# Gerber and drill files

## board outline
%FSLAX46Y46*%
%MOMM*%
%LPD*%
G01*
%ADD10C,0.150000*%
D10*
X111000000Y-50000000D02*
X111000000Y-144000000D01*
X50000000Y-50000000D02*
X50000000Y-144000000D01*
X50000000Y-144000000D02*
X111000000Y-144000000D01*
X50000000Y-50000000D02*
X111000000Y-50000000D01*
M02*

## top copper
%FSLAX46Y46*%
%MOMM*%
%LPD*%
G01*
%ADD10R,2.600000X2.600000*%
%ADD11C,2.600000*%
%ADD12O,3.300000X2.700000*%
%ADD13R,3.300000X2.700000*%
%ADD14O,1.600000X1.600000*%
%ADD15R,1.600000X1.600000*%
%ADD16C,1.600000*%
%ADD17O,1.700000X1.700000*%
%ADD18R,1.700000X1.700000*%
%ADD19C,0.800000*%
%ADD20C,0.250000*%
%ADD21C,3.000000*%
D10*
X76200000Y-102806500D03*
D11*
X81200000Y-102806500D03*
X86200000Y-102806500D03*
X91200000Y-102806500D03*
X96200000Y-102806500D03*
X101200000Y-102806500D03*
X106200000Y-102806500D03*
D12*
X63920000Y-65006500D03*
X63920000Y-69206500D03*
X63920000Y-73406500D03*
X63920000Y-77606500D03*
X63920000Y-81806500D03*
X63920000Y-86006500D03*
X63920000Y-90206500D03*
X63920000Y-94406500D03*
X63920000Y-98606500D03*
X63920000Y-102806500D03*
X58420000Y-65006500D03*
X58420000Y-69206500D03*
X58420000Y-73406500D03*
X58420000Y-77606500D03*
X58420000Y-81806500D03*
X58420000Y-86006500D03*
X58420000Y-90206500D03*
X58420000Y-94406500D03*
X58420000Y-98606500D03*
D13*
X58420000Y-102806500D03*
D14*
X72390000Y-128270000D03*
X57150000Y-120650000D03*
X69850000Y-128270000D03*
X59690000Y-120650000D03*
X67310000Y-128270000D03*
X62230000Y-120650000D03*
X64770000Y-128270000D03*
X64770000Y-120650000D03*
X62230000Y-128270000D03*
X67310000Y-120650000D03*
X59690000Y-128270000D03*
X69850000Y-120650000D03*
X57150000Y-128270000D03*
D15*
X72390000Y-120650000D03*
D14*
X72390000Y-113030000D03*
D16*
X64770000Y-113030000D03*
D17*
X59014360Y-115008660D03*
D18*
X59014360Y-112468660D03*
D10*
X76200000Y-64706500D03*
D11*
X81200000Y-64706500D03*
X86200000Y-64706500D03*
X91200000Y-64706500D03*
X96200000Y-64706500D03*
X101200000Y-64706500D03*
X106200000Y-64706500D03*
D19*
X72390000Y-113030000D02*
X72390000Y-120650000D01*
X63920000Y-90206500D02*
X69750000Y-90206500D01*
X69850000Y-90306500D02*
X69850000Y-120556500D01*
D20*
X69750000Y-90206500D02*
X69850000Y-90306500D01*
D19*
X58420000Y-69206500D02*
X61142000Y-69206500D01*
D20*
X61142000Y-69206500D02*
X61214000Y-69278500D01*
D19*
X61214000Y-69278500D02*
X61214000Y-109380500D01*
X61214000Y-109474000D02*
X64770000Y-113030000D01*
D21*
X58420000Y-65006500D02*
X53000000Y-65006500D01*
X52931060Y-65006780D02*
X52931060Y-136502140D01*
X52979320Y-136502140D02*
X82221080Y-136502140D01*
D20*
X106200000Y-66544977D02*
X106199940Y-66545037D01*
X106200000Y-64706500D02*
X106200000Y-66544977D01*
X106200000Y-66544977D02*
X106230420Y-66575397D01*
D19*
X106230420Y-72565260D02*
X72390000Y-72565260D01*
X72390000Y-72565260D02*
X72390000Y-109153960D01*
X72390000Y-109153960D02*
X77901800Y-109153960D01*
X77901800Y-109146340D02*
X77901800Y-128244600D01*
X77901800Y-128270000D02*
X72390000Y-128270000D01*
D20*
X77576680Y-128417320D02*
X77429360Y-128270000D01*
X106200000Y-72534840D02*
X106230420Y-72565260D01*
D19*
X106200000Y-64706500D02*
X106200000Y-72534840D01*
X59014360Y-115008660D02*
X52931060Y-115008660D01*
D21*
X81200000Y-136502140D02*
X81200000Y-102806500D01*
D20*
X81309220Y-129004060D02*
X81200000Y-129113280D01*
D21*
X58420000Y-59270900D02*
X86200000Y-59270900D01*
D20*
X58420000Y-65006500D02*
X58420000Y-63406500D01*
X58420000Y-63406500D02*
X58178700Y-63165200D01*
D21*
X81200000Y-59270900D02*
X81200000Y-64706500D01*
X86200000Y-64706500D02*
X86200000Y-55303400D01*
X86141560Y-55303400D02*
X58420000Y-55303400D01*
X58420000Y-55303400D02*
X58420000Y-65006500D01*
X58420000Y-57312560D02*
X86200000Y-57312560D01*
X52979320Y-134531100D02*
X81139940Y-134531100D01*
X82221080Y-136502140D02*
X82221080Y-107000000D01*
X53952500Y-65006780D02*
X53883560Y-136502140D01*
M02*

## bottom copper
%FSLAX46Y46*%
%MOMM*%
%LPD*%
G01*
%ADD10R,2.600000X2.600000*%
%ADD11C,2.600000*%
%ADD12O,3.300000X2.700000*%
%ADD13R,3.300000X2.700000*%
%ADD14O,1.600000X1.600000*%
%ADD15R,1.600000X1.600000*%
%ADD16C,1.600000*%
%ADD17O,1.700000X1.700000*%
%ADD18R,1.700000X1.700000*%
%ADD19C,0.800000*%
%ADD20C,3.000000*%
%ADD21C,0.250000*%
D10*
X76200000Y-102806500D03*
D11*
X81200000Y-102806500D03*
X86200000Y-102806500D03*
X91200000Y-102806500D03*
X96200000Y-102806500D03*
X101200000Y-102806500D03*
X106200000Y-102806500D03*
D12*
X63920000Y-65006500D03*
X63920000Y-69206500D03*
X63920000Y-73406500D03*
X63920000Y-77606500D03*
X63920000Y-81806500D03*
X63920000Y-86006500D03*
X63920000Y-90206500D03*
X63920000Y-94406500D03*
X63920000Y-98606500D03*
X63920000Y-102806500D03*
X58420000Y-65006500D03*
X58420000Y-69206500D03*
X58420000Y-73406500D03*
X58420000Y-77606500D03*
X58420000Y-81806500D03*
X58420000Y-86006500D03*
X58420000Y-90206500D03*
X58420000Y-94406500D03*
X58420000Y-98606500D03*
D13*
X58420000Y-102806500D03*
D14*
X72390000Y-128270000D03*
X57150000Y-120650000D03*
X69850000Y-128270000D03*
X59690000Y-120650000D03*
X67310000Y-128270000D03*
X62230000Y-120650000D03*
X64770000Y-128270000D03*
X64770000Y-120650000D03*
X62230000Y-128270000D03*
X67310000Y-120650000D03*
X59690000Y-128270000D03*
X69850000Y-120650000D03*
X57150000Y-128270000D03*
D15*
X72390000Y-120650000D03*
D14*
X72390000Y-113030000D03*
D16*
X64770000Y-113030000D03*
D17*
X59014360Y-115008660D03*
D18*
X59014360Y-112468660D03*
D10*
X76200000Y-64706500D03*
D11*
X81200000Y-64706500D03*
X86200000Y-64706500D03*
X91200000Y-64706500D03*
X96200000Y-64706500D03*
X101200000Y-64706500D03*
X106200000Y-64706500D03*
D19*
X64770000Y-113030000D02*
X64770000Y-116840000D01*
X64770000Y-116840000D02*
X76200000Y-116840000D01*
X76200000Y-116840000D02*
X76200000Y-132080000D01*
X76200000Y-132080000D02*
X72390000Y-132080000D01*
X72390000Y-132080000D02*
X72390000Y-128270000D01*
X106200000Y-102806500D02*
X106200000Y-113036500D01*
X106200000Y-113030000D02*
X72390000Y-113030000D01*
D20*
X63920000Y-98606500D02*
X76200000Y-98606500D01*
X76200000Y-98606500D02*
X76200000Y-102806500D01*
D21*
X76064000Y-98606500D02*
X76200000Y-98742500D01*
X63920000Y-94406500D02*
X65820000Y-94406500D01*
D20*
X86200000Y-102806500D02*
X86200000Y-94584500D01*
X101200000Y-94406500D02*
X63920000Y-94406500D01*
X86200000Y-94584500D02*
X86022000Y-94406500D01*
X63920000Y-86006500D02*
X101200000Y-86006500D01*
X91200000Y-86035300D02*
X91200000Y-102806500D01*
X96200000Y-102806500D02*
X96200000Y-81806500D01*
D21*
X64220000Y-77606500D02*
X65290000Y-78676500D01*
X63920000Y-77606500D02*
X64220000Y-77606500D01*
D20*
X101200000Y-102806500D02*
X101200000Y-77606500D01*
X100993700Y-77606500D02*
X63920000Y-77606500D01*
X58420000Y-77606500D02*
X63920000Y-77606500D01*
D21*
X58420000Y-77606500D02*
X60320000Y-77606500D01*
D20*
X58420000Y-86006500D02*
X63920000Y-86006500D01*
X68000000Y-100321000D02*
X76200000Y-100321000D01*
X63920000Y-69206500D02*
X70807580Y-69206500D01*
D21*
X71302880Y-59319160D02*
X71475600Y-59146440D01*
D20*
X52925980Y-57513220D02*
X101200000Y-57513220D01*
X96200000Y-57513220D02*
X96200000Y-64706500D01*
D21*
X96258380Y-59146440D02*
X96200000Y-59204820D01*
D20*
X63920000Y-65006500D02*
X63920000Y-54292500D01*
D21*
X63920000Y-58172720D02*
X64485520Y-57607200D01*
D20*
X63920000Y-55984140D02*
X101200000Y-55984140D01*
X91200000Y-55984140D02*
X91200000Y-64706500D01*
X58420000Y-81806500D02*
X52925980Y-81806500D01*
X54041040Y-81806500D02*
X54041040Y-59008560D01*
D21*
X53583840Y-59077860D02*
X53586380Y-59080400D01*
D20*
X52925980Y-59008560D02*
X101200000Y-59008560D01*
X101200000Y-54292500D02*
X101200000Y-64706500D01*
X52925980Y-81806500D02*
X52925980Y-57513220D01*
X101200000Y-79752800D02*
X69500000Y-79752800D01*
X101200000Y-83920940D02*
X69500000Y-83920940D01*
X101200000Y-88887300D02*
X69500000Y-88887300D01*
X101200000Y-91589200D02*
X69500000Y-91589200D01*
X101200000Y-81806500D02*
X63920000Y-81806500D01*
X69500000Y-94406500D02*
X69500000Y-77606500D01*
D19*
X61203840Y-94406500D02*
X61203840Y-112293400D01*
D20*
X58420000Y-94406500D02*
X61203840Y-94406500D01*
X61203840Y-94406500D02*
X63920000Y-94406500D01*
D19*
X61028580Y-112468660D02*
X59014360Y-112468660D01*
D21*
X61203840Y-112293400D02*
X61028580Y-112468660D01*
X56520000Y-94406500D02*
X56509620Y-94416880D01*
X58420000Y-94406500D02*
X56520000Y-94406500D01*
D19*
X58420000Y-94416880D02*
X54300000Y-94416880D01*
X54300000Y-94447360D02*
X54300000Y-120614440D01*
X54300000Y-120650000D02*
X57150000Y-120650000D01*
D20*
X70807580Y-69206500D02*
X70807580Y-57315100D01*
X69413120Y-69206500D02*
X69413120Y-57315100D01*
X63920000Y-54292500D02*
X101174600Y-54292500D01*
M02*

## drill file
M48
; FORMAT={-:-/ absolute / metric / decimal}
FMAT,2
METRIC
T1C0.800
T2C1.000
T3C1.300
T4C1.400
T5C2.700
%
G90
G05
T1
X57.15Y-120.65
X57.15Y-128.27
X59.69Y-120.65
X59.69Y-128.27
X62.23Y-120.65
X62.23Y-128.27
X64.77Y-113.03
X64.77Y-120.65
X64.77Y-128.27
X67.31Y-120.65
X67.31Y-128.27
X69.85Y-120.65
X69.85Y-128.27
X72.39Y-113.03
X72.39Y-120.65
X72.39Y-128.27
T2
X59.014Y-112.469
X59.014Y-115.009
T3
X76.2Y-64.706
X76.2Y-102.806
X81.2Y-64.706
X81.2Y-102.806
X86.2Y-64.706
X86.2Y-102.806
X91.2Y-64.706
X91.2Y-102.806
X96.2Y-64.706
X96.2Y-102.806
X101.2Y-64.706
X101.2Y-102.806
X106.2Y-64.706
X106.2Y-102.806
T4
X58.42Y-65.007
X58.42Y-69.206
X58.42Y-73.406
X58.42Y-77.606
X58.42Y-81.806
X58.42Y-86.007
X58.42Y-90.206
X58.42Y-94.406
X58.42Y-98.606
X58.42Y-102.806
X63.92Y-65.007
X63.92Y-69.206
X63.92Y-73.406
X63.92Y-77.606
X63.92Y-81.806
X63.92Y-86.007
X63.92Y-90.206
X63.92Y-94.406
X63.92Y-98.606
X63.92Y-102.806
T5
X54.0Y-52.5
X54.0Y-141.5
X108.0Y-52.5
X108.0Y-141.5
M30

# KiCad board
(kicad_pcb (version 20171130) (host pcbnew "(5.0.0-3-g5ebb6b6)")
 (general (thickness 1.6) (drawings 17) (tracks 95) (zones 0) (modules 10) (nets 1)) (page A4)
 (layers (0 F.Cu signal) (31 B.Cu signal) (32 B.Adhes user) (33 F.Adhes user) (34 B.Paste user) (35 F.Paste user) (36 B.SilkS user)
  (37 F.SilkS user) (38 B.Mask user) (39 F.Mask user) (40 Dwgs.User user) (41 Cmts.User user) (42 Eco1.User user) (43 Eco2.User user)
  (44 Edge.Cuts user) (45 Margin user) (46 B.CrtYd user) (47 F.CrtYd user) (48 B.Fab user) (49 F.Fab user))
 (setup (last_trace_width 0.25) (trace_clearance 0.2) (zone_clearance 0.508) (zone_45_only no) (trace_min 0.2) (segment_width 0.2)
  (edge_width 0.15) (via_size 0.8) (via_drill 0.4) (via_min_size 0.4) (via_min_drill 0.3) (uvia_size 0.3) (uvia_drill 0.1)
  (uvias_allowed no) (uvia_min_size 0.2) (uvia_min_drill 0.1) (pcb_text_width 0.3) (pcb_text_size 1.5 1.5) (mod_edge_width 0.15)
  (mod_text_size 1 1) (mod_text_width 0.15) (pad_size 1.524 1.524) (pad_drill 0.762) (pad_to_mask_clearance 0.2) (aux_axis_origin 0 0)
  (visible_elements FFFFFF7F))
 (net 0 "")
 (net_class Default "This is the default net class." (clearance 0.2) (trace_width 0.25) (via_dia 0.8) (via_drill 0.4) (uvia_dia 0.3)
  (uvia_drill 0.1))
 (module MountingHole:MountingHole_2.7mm (layer F.Cu) (at 54 52.5)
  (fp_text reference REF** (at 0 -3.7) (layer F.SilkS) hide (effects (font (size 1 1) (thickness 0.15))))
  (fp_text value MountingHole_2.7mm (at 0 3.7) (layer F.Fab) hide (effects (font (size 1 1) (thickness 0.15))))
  (pad 1 np_thru_hole circle (at 0 0) (size 2.7 2.7) (drill 2.7) (layers *.Cu *.Mask)))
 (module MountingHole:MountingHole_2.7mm (layer F.Cu) (at 54 141.5)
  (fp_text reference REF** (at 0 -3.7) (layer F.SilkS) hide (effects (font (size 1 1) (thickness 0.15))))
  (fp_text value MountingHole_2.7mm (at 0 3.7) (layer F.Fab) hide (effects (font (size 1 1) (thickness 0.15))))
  (pad 1 np_thru_hole circle (at 0 0) (size 2.7 2.7) (drill 2.7) (layers *.Cu *.Mask)))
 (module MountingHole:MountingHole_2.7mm (layer F.Cu) (at 108 141.5)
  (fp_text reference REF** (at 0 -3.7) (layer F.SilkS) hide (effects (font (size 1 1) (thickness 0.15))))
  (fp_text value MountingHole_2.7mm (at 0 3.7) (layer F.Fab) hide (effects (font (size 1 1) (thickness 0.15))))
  (pad 1 np_thru_hole circle (at 0 0) (size 2.7 2.7) (drill 2.7) (layers *.Cu *.Mask)))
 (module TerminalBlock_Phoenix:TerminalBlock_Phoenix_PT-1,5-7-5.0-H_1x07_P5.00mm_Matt (layer F.Cu) (at 76.2 102.8065)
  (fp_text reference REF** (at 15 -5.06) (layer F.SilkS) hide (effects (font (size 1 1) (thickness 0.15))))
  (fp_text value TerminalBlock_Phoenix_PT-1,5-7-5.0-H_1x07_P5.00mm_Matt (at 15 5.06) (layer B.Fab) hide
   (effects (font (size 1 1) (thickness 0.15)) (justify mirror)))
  (pad 1 thru_hole rect (at 0 0) (size 2.6 2.6) (drill 1.3) (layers *.Cu *.Mask))
  (pad 2 thru_hole circle (at 5 0) (size 2.6 2.6) (drill 1.3) (layers *.Cu *.Mask))
  (pad 3 thru_hole circle (at 10 0) (size 2.6 2.6) (drill 1.3) (layers *.Cu *.Mask))
  (pad 4 thru_hole circle (at 15 0) (size 2.6 2.6) (drill 1.3) (layers *.Cu *.Mask))
  (pad 5 thru_hole circle (at 20 0) (size 2.6 2.6) (drill 1.3) (layers *.Cu *.Mask))
  (pad 6 thru_hole circle (at 25 0) (size 2.6 2.6) (drill 1.3) (layers *.Cu *.Mask))
  (pad 7 thru_hole circle (at 30 0) (size 2.6 2.6) (drill 1.3) (layers *.Cu *.Mask)))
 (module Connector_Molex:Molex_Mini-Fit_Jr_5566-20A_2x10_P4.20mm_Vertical (layer F.Cu) (at 58.42 102.8065 90)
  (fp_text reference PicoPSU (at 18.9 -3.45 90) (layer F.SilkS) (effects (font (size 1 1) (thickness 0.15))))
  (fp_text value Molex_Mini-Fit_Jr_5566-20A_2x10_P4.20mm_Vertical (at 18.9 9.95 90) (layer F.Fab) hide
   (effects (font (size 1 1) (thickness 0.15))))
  (pad 20 thru_hole oval (at 37.8 5.5 90) (size 2.7 3.3) (drill 1.4) (layers *.Cu *.Mask))
  (pad 19 thru_hole oval (at 33.6 5.5 90) (size 2.7 3.3) (drill 1.4) (layers *.Cu *.Mask))
  (pad 18 thru_hole oval (at 29.4 5.5 90) (size 2.7 3.3) (drill 1.4) (layers *.Cu *.Mask))
  (pad 17 thru_hole oval (at 25.2 5.5 90) (size 2.7 3.3) (drill 1.4) (layers *.Cu *.Mask))
  (pad 16 thru_hole oval (at 21 5.5 90) (size 2.7 3.3) (drill 1.4) (layers *.Cu *.Mask))
  (pad 15 thru_hole oval (at 16.8 5.5 90) (size 2.7 3.3) (drill 1.4) (layers *.Cu *.Mask))
  (pad 14 thru_hole oval (at 12.6 5.5 90) (size 2.7 3.3) (drill 1.4) (layers *.Cu *.Mask))
  (pad 13 thru_hole oval (at 8.4 5.5 90) (size 2.7 3.3) (drill 1.4) (layers *.Cu *.Mask))
  (pad 12 thru_hole oval (at 4.2 5.5 90) (size 2.7 3.3) (drill 1.4) (layers *.Cu *.Mask))
  (pad 11 thru_hole oval (at 0 5.5 90) (size 2.7 3.3) (drill 1.4) (layers *.Cu *.Mask))
  (pad 10 thru_hole oval (at 37.8 0 90) (size 2.7 3.3) (drill 1.4) (layers *.Cu *.Mask))
  (pad 9 thru_hole oval (at 33.6 0 90) (size 2.7 3.3) (drill 1.4) (layers *.Cu *.Mask))
  (pad 8 thru_hole oval (at 29.4 0 90) (size 2.7 3.3) (drill 1.4) (layers *.Cu *.Mask))
  (pad 7 thru_hole oval (at 25.2 0 90) (size 2.7 3.3) (drill 1.4) (layers *.Cu *.Mask))
  (pad 6 thru_hole oval (at 21 0 90) (size 2.7 3.3) (drill 1.4) (layers *.Cu *.Mask))
  (pad 5 thru_hole oval (at 16.8 0 90) (size 2.7 3.3) (drill 1.4) (layers *.Cu *.Mask))
  (pad 4 thru_hole oval (at 12.6 0 90) (size 2.7 3.3) (drill 1.4) (layers *.Cu *.Mask))
  (pad 3 thru_hole oval (at 8.4 0 90) (size 2.7 3.3) (drill 1.4) (layers *.Cu *.Mask))
  (pad 2 thru_hole oval (at 4.2 0 90) (size 2.7 3.3) (drill 1.4) (layers *.Cu *.Mask))
  (pad 1 thru_hole rect (at 0 0 90) (size 2.7 3.3) (drill 1.4) (layers *.Cu *.Mask)))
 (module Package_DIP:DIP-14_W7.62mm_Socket (layer F.Cu) (at 72.39 120.65 270)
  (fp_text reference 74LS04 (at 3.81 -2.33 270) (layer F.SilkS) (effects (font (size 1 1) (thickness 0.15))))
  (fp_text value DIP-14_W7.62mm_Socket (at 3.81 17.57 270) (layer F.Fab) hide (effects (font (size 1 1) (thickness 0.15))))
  (pad 14 thru_hole oval (at 7.62 0 270) (size 1.6 1.6) (drill 0.8) (layers *.Cu *.Mask))
  (pad 7 thru_hole oval (at 0 15.24 270) (size 1.6 1.6) (drill 0.8) (layers *.Cu *.Mask))
  (pad 13 thru_hole oval (at 7.62 2.54 270) (size 1.6 1.6) (drill 0.8) (layers *.Cu *.Mask))
  (pad 6 thru_hole oval (at 0 12.7 270) (size 1.6 1.6) (drill 0.8) (layers *.Cu *.Mask))
  (pad 12 thru_hole oval (at 7.62 5.08 270) (size 1.6 1.6) (drill 0.8) (layers *.Cu *.Mask))
  (pad 5 thru_hole oval (at 0 10.16 270) (size 1.6 1.6) (drill 0.8) (layers *.Cu *.Mask))
  (pad 11 thru_hole oval (at 7.62 7.62 270) (size 1.6 1.6) (drill 0.8) (layers *.Cu *.Mask))
  (pad 4 thru_hole oval (at 0 7.62 270) (size 1.6 1.6) (drill 0.8) (layers *.Cu *.Mask))
  (pad 10 thru_hole oval (at 7.62 10.16 270) (size 1.6 1.6) (drill 0.8) (layers *.Cu *.Mask))
  (pad 3 thru_hole oval (at 0 5.08 270) (size 1.6 1.6) (drill 0.8) (layers *.Cu *.Mask))
  (pad 9 thru_hole oval (at 7.62 12.7 270) (size 1.6 1.6) (drill 0.8) (layers *.Cu *.Mask))
  (pad 2 thru_hole oval (at 0 2.54 270) (size 1.6 1.6) (drill 0.8) (layers *.Cu *.Mask))
  (pad 8 thru_hole oval (at 7.62 15.24 270) (size 1.6 1.6) (drill 0.8) (layers *.Cu *.Mask))
  (pad 1 thru_hole rect (at 0 0 270) (size 1.6 1.6) (drill 0.8) (layers *.Cu *.Mask)))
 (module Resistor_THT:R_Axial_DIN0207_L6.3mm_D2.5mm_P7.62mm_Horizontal (layer F.Cu) (at 64.77 113.03)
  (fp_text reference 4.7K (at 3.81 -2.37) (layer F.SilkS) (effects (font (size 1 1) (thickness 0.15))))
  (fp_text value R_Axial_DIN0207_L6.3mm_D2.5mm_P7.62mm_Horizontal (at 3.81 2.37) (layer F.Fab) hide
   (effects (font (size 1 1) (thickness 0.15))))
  (pad 2 thru_hole oval (at 7.62 0) (size 1.6 1.6) (drill 0.8) (layers *.Cu *.Mask))
  (pad 1 thru_hole circle (at 0 0) (size 1.6 1.6) (drill 0.8) (layers *.Cu *.Mask)))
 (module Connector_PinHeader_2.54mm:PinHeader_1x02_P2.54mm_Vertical (layer F.Cu) (at 59.01436 112.46866)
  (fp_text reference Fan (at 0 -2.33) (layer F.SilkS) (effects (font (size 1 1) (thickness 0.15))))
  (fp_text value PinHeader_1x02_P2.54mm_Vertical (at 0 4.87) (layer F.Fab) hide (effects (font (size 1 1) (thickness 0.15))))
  (pad 2 thru_hole oval (at 0 2.54) (size 1.7 1.7) (drill 1) (layers *.Cu *.Mask))
  (pad 1 thru_hole rect (at 0 0) (size 1.7 1.7) (drill 1) (layers *.Cu *.Mask)))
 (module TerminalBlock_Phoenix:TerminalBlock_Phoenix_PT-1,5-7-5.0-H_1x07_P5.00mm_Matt (layer F.Cu) (at 76.2 64.7065)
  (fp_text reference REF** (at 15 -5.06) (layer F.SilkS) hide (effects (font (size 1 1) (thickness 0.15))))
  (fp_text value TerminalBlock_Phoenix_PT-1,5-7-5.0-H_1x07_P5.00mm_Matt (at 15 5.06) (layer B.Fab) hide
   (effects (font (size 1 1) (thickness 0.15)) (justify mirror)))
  (pad 1 thru_hole rect (at 0 0) (size 2.6 2.6) (drill 1.3) (layers *.Cu *.Mask))
  (pad 2 thru_hole circle (at 5 0) (size 2.6 2.6) (drill 1.3) (layers *.Cu *.Mask))
  (pad 3 thru_hole circle (at 10 0) (size 2.6 2.6) (drill 1.3) (layers *.Cu *.Mask))
  (pad 4 thru_hole circle (at 15 0) (size 2.6 2.6) (drill 1.3) (layers *.Cu *.Mask))
  (pad 5 thru_hole circle (at 20 0) (size 2.6 2.6) (drill 1.3) (layers *.Cu *.Mask))
  (pad 6 thru_hole circle (at 25 0) (size 2.6 2.6) (drill 1.3) (layers *.Cu *.Mask))
  (pad 7 thru_hole circle (at 30 0) (size 2.6 2.6) (drill 1.3) (layers *.Cu *.Mask)))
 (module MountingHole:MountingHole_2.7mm (layer F.Cu) (at 108 52.5)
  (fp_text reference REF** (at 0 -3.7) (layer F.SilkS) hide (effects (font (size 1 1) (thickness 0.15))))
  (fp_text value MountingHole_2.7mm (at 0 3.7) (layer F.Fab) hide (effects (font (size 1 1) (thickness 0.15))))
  (pad 1 np_thru_hole circle (at 0 0) (size 2.7 2.7) (drill 2.7) (layers *.Cu *.Mask)))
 (gr_line (start 111 50) (end 111 144) (layer Edge.Cuts) (width 0.15))
 (gr_line (start 50 50) (end 50 144) (layer Edge.Cuts) (width 0.15))
 (gr_line (start 50 144) (end 111 144) (layer Edge.Cuts) (width 0.15))
 (gr_line (start 50 50) (end 111 50) (layer Edge.Cuts) (width 0.15))
 (segment (start 72.39 113.03) (end 72.39 120.65) (width 0.8) (layer F.Cu) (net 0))
 (segment (start 63.92 90.2065) (end 69.75 90.2065) (width 0.8) (layer F.Cu) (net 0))
 (segment (start 69.85 90.3065) (end 69.85 120.5565) (width 0.8) (layer F.Cu) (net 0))
 (segment (start 69.75 90.2065) (end 69.85 90.3065) (width 0.25) (layer F.Cu) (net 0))
 (segment (start 64.77 113.03) (end 64.77 116.84) (width 0.8) (layer B.Cu) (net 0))
 (segment (start 64.77 116.84) (end 76.2 116.84) (width 0.8) (layer B.Cu) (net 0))
 (segment (start 76.2 116.84) (end 76.2 132.08) (width 0.8) (layer B.Cu) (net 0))
 (segment (start 76.2 132.08) (end 72.39 132.08) (width 0.8) (layer B.Cu) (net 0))
 (segment (start 72.39 132.08) (end 72.39 128.27) (width 0.8) (layer B.Cu) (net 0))
 (segment (start 106.2 102.8065) (end 106.2 113.0365) (width 0.8) (layer B.Cu) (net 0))
 (segment (start 106.2 113.03) (end 72.39 113.03) (width 0.8) (layer B.Cu) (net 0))
 (segment (start 58.42 69.2065) (end 61.142 69.2065) (width 0.8) (layer F.Cu) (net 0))
 (segment (start 61.142 69.2065) (end 61.214 69.2785) (width 0.25) (layer F.Cu) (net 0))
 (segment (start 61.214 69.2785) (end 61.214 109.3805) (width 0.8) (layer F.Cu) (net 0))
 (segment (start 61.214 109.474) (end 64.77 113.03) (width 0.8) (layer F.Cu) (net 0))
 (segment (start 63.92 98.6065) (end 76.2 98.6065) (width 3) (layer B.Cu) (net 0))
 (segment (start 76.2 98.6065) (end 76.2 102.8065) (width 3) (layer B.Cu) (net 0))
 (segment (start 76.064 98.6065) (end 76.2 98.7425) (width 0.25) (layer B.Cu) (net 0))
 (segment (start 63.92 94.4065) (end 65.82 94.4065) (width 0.25) (layer B.Cu) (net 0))
 (segment (start 86.2 102.8065) (end 86.2 94.5845) (width 3) (layer B.Cu) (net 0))
 (segment (start 101.2 94.4065) (end 63.92 94.4065) (width 3) (layer B.Cu) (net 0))
 (segment (start 86.2 94.5845) (end 86.022 94.4065) (width 3) (layer B.Cu) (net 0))
 (segment (start 63.92 86.0065) (end 101.2 86.0065) (width 3) (layer B.Cu) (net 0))
 (segment (start 91.2 86.0353) (end 91.2 102.8065) (width 3) (layer B.Cu) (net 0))
 (segment (start 96.2 102.8065) (end 96.2 81.8065) (width 3) (layer B.Cu) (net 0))
 (segment (start 64.22 77.6065) (end 65.29 78.6765) (width 0.25) (layer B.Cu) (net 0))
 (segment (start 63.92 77.6065) (end 64.22 77.6065) (width 0.25) (layer B.Cu) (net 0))
 (segment (start 101.2 102.8065) (end 101.2 77.6065) (width 3) (layer B.Cu) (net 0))
 (segment (start 100.9937 77.6065) (end 63.92 77.6065) (width 3) (layer B.Cu) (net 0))
 (segment (start 58.42 65.0065) (end 53 65.0065) (width 3) (layer F.Cu) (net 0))
 (segment (start 52.93106 65.00678) (end 52.93106 136.50214) (width 3) (layer F.Cu) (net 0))
 (segment (start 52.97932 136.50214) (end 82.22108 136.50214) (width 3) (layer F.Cu) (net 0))
 (segment (start 106.2 66.544977) (end 106.19994 66.545037) (width 0.25) (layer F.Cu) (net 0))
 (segment (start 106.2 64.7065) (end 106.2 66.544977) (width 0.25) (layer F.Cu) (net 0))
 (segment (start 106.2 66.544977) (end 106.23042 66.575397) (width 0.25) (layer F.Cu) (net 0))
 (segment (start 106.23042 72.56526) (end 72.39 72.56526) (width 0.8) (layer F.Cu) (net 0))
 (segment (start 72.39 72.56526) (end 72.39 109.15396) (width 0.8) (layer F.Cu) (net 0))
 (segment (start 72.39 109.15396) (end 77.9018 109.15396) (width 0.8) (layer F.Cu) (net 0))
 (segment (start 77.9018 109.14634) (end 77.9018 128.2446) (width 0.8) (layer F.Cu) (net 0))
 (segment (start 77.9018 128.27) (end 72.39 128.27) (width 0.8) (layer F.Cu) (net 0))
 (segment (start 77.57668 128.41732) (end 77.42936 128.27) (width 0.25) (layer F.Cu) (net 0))
 (segment (start 106.2 72.53484) (end 106.23042 72.56526) (width 0.25) (layer F.Cu) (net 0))
 (segment (start 106.2 64.7065) (end 106.2 72.53484) (width 0.8) (layer F.Cu) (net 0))
 (segment (start 59.01436 115.00866) (end 52.93106 115.00866) (width 0.8) (layer F.Cu) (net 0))
 (segment (start 81.2 136.50214) (end 81.2 102.8065) (width 3) (layer F.Cu) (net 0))
 (segment (start 81.30922 129.00406) (end 81.2 129.11328) (width 0.25) (layer F.Cu) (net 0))
 (segment (start 58.42 59.2709) (end 86.2 59.2709) (width 3) (layer F.Cu) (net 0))
 (segment (start 58.42 65.0065) (end 58.42 63.4065) (width 0.25) (layer F.Cu) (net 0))
 (segment (start 58.42 63.4065) (end 58.1787 63.1652) (width 0.25) (layer F.Cu) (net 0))
 (segment (start 81.2 59.2709) (end 81.2 64.7065) (width 3) (layer F.Cu) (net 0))
 (segment (start 86.2 64.7065) (end 86.2 55.3034) (width 3) (layer F.Cu) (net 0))
 (segment (start 86.14156 55.3034) (end 58.42 55.3034) (width 3) (layer F.Cu) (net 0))
 (segment (start 58.42 55.3034) (end 58.42 65.0065) (width 3) (layer F.Cu) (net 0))
 (segment (start 58.42 57.31256) (end 86.2 57.31256) (width 3) (layer F.Cu) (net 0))
 (segment (start 52.97932 134.5311) (end 81.13994 134.5311) (width 3) (layer F.Cu) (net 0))
 (segment (start 82.22108 136.50214) (end 82.22108 107) (width 3) (layer F.Cu) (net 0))
 (segment (start 53.9525 65.00678) (end 53.88356 136.50214) (width 3) (layer F.Cu) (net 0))
 (segment (start 58.42 77.6065) (end 63.92 77.6065) (width 3) (layer B.Cu) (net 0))
 (segment (start 58.42 77.6065) (end 60.32 77.6065) (width 0.25) (layer B.Cu) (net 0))
 (segment (start 58.42 86.0065) (end 63.92 86.0065) (width 3) (layer B.Cu) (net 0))
 (segment (start 68 100.321) (end 76.2 100.321) (width 3) (layer B.Cu) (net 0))
 (segment (start 63.92 69.2065) (end 70.80758 69.2065) (width 3) (layer B.Cu) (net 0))
 (segment (start 71.30288 59.31916) (end 71.4756 59.14644) (width 0.25) (layer B.Cu) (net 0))
 (segment (start 52.92598 57.51322) (end 101.2 57.51322) (width 3) (layer B.Cu) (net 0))
 (segment (start 96.2 57.51322) (end 96.2 64.7065) (width 3) (layer B.Cu) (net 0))
 (segment (start 96.25838 59.14644) (end 96.2 59.20482) (width 0.25) (layer B.Cu) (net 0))
 (segment (start 63.92 65.0065) (end 63.92 54.2925) (width 3) (layer B.Cu) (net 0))
 (segment (start 63.92 58.17272) (end 64.48552 57.6072) (width 0.25) (layer B.Cu) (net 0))
 (segment (start 63.92 55.98414) (end 101.2 55.98414) (width 3) (layer B.Cu) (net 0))
 (segment (start 91.2 55.98414) (end 91.2 64.7065) (width 3) (layer B.Cu) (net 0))
 (segment (start 58.42 81.8065) (end 52.92598 81.8065) (width 3) (layer B.Cu) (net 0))
 (segment (start 54.04104 81.8065) (end 54.04104 59.00856) (width 3) (layer B.Cu) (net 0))
 (segment (start 53.58384 59.07786) (end 53.58638 59.0804) (width 0.25) (layer B.Cu) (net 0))
 (segment (start 52.92598 59.00856) (end 101.2 59.00856) (width 3) (layer B.Cu) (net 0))
 (segment (start 101.2 54.2925) (end 101.2 64.7065) (width 3) (layer B.Cu) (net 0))
 (segment (start 52.92598 81.8065) (end 52.92598 57.51322) (width 3) (layer B.Cu) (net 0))
 (segment (start 101.2 79.7528) (end 69.5 79.7528) (width 3) (layer B.Cu) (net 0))
 (segment (start 101.2 83.92094) (end 69.5 83.92094) (width 3) (layer B.Cu) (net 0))
 (segment (start 101.2 88.8873) (end 69.5 88.8873) (width 3) (layer B.Cu) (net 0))
 (segment (start 101.2 91.5892) (end 69.5 91.5892) (width 3) (layer B.Cu) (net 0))
 (segment (start 101.2 81.8065) (end 63.92 81.8065) (width 3) (layer B.Cu) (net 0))
 (segment (start 69.5 94.4065) (end 69.5 77.6065) (width 3) (layer B.Cu) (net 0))
 (segment (start 61.20384 94.4065) (end 61.20384 112.2934) (width 0.8) (layer B.Cu) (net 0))
 (segment (start 58.42 94.4065) (end 61.20384 94.4065) (width 3) (layer B.Cu) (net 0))
 (segment (start 61.20384 94.4065) (end 63.92 94.4065) (width 3) (layer B.Cu) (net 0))
 (segment (start 61.02858 112.46866) (end 59.01436 112.46866) (width 0.8) (layer B.Cu) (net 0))
 (segment (start 61.20384 112.2934) (end 61.02858 112.46866) (width 0.25) (layer B.Cu) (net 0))
 (segment (start 56.52 94.4065) (end 56.50962 94.41688) (width 0.25) (layer B.Cu) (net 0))
 (segment (start 58.42 94.4065) (end 56.52 94.4065) (width 0.25) (layer B.Cu) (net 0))
 (segment (start 58.42 94.41688) (end 54.3 94.41688) (width 0.8) (layer B.Cu) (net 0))
 (segment (start 54.3 94.44736) (end 54.3 120.61444) (width 0.8) (layer B.Cu) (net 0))
 (segment (start 54.3 120.65) (end 57.15 120.65) (width 0.8) (layer B.Cu) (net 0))
 (segment (start 70.80758 69.2065) (end 70.80758 57.3151) (width 3) (layer B.Cu) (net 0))
 (segment (start 69.41312 69.2065) (end 69.41312 57.3151) (width 3) (layer B.Cu) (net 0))
 (segment (start 63.92 54.2925) (end 101.1746 54.2925) (width 3) (layer B.Cu) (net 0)))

